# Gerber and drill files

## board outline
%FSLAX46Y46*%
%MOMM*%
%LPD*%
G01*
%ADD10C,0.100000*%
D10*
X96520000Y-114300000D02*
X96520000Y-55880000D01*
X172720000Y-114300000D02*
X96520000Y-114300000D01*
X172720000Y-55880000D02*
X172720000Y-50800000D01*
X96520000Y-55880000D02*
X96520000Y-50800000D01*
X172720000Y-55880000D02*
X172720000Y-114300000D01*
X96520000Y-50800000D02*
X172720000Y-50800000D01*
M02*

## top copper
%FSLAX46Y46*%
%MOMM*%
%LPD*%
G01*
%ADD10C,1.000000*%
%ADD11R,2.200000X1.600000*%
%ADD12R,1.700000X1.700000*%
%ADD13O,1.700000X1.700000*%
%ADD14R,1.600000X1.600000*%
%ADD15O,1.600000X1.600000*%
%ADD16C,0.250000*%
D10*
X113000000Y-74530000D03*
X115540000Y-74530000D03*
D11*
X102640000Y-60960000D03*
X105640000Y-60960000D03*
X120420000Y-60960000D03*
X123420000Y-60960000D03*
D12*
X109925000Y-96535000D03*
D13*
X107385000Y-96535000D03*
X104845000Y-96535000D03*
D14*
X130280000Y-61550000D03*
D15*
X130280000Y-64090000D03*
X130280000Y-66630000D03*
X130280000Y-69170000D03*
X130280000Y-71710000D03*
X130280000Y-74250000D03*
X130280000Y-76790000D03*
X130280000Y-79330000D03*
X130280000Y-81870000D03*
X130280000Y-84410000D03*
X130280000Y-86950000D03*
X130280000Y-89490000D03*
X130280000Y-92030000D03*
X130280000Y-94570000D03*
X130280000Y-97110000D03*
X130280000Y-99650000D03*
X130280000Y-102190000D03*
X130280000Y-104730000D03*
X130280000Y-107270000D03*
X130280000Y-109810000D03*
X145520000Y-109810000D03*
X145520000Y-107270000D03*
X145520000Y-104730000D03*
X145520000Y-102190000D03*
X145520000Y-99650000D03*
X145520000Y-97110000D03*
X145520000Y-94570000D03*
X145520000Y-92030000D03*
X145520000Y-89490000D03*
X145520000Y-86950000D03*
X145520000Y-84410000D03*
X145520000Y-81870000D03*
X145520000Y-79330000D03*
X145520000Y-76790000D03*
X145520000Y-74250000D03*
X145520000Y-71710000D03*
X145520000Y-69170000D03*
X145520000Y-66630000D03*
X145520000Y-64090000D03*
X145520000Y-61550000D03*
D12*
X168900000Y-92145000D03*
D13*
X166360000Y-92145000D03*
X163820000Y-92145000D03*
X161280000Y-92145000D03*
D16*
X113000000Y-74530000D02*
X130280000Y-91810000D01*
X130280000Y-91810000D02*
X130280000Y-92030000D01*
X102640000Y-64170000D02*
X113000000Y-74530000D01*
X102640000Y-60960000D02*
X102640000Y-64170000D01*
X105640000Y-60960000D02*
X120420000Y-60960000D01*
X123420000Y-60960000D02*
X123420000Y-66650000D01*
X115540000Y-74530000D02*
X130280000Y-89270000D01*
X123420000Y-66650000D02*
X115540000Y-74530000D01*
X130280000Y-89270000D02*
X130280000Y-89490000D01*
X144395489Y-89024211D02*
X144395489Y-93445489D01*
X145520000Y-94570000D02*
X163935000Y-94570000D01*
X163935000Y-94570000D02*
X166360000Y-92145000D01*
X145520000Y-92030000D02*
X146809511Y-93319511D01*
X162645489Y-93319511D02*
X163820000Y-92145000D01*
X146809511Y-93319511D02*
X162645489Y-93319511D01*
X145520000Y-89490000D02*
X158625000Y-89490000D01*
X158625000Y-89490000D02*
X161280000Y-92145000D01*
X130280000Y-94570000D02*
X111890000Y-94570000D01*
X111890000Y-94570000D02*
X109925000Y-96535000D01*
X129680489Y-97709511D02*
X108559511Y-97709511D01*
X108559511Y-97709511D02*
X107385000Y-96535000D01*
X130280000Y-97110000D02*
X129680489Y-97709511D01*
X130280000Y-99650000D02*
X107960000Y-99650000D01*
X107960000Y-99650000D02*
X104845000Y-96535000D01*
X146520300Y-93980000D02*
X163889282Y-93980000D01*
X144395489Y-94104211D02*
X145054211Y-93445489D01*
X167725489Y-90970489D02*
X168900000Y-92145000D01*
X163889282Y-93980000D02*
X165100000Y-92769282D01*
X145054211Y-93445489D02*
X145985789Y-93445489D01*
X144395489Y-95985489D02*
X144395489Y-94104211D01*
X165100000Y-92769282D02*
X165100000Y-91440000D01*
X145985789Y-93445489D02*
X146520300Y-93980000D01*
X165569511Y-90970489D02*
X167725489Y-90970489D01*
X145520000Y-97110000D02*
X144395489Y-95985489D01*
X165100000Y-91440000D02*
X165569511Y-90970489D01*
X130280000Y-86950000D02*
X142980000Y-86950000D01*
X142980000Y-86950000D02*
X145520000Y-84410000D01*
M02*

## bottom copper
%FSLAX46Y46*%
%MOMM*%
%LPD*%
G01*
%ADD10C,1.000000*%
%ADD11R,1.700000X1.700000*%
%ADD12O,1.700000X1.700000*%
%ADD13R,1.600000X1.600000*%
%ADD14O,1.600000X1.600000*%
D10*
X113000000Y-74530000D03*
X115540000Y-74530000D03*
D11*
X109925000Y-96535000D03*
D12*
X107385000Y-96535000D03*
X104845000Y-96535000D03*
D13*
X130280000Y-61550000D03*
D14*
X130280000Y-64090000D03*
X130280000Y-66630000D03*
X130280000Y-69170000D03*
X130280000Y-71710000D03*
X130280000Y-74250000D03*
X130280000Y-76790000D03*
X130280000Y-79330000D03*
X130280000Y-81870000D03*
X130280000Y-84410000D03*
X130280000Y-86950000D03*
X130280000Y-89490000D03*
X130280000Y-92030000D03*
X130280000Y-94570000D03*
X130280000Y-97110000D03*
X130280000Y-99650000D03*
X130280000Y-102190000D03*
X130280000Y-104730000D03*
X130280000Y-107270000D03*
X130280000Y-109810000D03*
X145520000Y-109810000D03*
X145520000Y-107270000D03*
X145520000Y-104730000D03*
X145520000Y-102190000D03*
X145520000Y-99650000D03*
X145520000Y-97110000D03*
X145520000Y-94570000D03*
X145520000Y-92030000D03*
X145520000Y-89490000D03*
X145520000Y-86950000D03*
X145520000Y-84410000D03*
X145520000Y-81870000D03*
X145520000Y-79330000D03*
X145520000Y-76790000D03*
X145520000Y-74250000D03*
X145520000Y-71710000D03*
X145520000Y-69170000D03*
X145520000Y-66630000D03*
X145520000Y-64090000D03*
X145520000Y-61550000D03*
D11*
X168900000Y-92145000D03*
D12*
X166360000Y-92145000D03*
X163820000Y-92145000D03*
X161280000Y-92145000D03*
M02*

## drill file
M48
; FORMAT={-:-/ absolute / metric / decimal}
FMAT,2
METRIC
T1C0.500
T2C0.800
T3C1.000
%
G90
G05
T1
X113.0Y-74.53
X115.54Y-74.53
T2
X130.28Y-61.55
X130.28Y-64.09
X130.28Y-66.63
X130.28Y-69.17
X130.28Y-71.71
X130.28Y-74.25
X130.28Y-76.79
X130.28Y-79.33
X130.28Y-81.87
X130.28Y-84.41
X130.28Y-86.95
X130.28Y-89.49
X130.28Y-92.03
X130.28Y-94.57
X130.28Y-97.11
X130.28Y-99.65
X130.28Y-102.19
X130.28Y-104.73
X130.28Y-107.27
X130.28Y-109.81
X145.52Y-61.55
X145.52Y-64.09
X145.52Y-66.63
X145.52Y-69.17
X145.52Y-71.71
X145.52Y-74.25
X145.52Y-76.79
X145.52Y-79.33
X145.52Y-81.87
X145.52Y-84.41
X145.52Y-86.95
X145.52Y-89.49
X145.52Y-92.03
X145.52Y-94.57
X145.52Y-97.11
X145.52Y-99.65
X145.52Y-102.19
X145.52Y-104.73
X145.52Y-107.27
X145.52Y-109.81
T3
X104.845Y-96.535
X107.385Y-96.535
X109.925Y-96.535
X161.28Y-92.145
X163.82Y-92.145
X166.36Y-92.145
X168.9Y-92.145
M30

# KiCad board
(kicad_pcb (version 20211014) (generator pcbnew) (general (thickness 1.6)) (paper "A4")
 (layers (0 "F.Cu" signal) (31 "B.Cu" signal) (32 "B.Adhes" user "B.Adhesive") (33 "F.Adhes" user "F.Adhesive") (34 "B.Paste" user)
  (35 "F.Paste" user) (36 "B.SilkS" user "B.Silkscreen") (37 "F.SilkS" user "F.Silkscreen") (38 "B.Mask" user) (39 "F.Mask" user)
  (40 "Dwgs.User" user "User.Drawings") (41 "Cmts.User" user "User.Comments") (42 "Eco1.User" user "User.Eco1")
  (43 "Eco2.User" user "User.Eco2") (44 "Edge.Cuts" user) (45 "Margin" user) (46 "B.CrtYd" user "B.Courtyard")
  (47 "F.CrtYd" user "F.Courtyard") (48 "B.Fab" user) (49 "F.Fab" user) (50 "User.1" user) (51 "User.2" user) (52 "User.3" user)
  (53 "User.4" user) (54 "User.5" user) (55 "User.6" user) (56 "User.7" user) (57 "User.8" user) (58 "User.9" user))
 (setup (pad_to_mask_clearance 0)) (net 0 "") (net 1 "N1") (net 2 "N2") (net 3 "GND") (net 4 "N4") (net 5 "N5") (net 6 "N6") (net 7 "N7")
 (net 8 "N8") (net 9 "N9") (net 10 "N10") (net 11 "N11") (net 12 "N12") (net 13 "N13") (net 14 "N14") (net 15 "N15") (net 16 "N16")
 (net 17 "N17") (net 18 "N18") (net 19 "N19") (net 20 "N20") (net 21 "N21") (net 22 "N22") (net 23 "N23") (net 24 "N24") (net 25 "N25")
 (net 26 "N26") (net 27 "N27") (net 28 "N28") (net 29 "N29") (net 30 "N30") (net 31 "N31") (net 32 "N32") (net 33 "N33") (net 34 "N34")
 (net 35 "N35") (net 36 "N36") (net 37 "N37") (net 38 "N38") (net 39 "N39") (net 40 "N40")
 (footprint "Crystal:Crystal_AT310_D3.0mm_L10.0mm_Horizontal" (layer "F.Cu") (at 113 74.53)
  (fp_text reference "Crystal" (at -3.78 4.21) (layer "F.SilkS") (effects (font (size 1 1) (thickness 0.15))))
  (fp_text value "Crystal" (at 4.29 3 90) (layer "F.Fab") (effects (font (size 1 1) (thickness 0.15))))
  (pad "1" thru_hole circle (at 0 0) (size 1 1) (drill 0.5) (layers *.Cu *.Mask) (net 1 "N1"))
  (pad "2" thru_hole circle (at 2.54 0) (size 1 1) (drill 0.5) (layers *.Cu *.Mask) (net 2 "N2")))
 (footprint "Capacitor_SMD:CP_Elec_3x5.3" (layer "F.Cu") (at 104.14 60.96)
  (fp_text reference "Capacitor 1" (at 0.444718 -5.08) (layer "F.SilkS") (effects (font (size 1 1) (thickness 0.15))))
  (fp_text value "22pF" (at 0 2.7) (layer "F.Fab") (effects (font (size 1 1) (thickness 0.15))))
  (pad "1" smd rect (at -1.5 0) (size 2.2 1.6) (layers "F.Cu" "F.Paste" "F.Mask") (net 1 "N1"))
  (pad "2" smd rect (at 1.5 0) (size 2.2 1.6) (layers "F.Cu" "F.Paste" "F.Mask") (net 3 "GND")))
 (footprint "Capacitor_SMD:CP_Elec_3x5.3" (layer "F.Cu") (at 121.92 60.96)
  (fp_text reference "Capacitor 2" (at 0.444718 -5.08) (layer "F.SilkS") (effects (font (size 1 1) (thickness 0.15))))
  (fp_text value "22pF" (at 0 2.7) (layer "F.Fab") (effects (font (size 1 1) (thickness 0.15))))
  (pad "1" smd rect (at -1.5 0) (size 2.2 1.6) (layers "F.Cu" "F.Paste" "F.Mask") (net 3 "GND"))
  (pad "2" smd rect (at 1.5 0) (size 2.2 1.6) (layers "F.Cu" "F.Paste" "F.Mask") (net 2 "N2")))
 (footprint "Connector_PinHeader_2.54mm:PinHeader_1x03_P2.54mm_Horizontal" (layer "F.Cu") (at 109.925 96.535 -90)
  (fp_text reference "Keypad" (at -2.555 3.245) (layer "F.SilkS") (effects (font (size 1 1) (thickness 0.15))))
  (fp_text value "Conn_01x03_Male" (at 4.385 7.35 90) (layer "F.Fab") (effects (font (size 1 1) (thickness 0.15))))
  (pad "1" thru_hole rect (at 0 0 270) (size 1.7 1.7) (drill 1) (layers *.Cu *.Mask) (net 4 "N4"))
  (pad "2" thru_hole oval (at 0 2.54 270) (size 1.7 1.7) (drill 1) (layers *.Cu *.Mask) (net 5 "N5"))
  (pad "3" thru_hole oval (at 0 5.08 270) (size 1.7 1.7) (drill 1) (layers *.Cu *.Mask) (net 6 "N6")))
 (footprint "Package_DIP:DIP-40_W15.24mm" (layer "F.Cu") (at 130.28 61.55)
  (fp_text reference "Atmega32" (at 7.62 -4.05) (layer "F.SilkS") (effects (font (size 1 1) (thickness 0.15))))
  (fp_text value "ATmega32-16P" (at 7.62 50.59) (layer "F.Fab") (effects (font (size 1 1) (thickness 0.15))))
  (pad "1" thru_hole rect (at 0 0) (size 1.6 1.6) (drill 0.8) (layers *.Cu *.Mask) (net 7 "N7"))
  (pad "2" thru_hole oval (at 0 2.54) (size 1.6 1.6) (drill 0.8) (layers *.Cu *.Mask) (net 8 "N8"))
  (pad "3" thru_hole oval (at 0 5.08) (size 1.6 1.6) (drill 0.8) (layers *.Cu *.Mask) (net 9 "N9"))
  (pad "4" thru_hole oval (at 0 7.62) (size 1.6 1.6) (drill 0.8) (layers *.Cu *.Mask) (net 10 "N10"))
  (pad "5" thru_hole oval (at 0 10.16) (size 1.6 1.6) (drill 0.8) (layers *.Cu *.Mask) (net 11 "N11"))
  (pad "6" thru_hole oval (at 0 12.7) (size 1.6 1.6) (drill 0.8) (layers *.Cu *.Mask) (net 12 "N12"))
  (pad "7" thru_hole oval (at 0 15.24) (size 1.6 1.6) (drill 0.8) (layers *.Cu *.Mask) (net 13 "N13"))
  (pad "8" thru_hole oval (at 0 17.78) (size 1.6 1.6) (drill 0.8) (layers *.Cu *.Mask) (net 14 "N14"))
  (pad "9" thru_hole oval (at 0 20.32) (size 1.6 1.6) (drill 0.8) (layers *.Cu *.Mask) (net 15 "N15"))
  (pad "10" thru_hole oval (at 0 22.86) (size 1.6 1.6) (drill 0.8) (layers *.Cu *.Mask) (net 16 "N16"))
  (pad "11" thru_hole oval (at 0 25.4) (size 1.6 1.6) (drill 0.8) (layers *.Cu *.Mask) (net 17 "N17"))
  (pad "12" thru_hole oval (at 0 27.94) (size 1.6 1.6) (drill 0.8) (layers *.Cu *.Mask) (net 2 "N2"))
  (pad "13" thru_hole oval (at 0 30.48) (size 1.6 1.6) (drill 0.8) (layers *.Cu *.Mask) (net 1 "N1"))
  (pad "14" thru_hole oval (at 0 33.02) (size 1.6 1.6) (drill 0.8) (layers *.Cu *.Mask) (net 4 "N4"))
  (pad "15" thru_hole oval (at 0 35.56) (size 1.6 1.6) (drill 0.8) (layers *.Cu *.Mask) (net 5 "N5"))
  (pad "16" thru_hole oval (at 0 38.1) (size 1.6 1.6) (drill 0.8) (layers *.Cu *.Mask) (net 6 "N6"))
  (pad "17" thru_hole oval (at 0 40.64) (size 1.6 1.6) (drill 0.8) (layers *.Cu *.Mask) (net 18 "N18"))
  (pad "18" thru_hole oval (at 0 43.18) (size 1.6 1.6) (drill 0.8) (layers *.Cu *.Mask) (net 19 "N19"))
  (pad "19" thru_hole oval (at 0 45.72) (size 1.6 1.6) (drill 0.8) (layers *.Cu *.Mask) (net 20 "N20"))
  (pad "20" thru_hole oval (at 0 48.26) (size 1.6 1.6) (drill 0.8) (layers *.Cu *.Mask) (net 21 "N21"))
  (pad "21" thru_hole oval (at 15.24 48.26) (size 1.6 1.6) (drill 0.8) (layers *.Cu *.Mask) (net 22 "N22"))
  (pad "22" thru_hole oval (at 15.24 45.72) (size 1.6 1.6) (drill 0.8) (layers *.Cu *.Mask) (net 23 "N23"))
  (pad "23" thru_hole oval (at 15.24 43.18) (size 1.6 1.6) (drill 0.8) (layers *.Cu *.Mask) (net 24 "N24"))
  (pad "24" thru_hole oval (at 15.24 40.64) (size 1.6 1.6) (drill 0.8) (layers *.Cu *.Mask) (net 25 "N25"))
  (pad "25" thru_hole oval (at 15.24 38.1) (size 1.6 1.6) (drill 0.8) (layers *.Cu *.Mask) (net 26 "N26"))
  (pad "26" thru_hole oval (at 15.24 35.56) (size 1.6 1.6) (drill 0.8) (layers *.Cu *.Mask) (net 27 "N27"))
  (pad "27" thru_hole oval (at 15.24 33.02) (size 1.6 1.6) (drill 0.8) (layers *.Cu *.Mask) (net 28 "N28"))
  (pad "28" thru_hole oval (at 15.24 30.48) (size 1.6 1.6) (drill 0.8) (layers *.Cu *.Mask) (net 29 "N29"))
  (pad "29" thru_hole oval (at 15.24 27.94) (size 1.6 1.6) (drill 0.8) (layers *.Cu *.Mask) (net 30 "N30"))
  (pad "30" thru_hole oval (at 15.24 25.4) (size 1.6 1.6) (drill 0.8) (layers *.Cu *.Mask) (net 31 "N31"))
  (pad "31" thru_hole oval (at 15.24 22.86) (size 1.6 1.6) (drill 0.8) (layers *.Cu *.Mask) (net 17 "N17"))
  (pad "32" thru_hole oval (at 15.24 20.32) (size 1.6 1.6) (drill 0.8) (layers *.Cu *.Mask) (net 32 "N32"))
  (pad "33" thru_hole oval (at 15.24 17.78) (size 1.6 1.6) (drill 0.8) (layers *.Cu *.Mask) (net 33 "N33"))
  (pad "34" thru_hole oval (at 15.24 15.24) (size 1.6 1.6) (drill 0.8) (layers *.Cu *.Mask) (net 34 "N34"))
  (pad "35" thru_hole oval (at 15.24 12.7) (size 1.6 1.6) (drill 0.8) (layers *.Cu *.Mask) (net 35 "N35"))
  (pad "36" thru_hole oval (at 15.24 10.16) (size 1.6 1.6) (drill 0.8) (layers *.Cu *.Mask) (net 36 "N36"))
  (pad "37" thru_hole oval (at 15.24 7.62) (size 1.6 1.6) (drill 0.8) (layers *.Cu *.Mask) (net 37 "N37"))
  (pad "38" thru_hole oval (at 15.24 5.08) (size 1.6 1.6) (drill 0.8) (layers *.Cu *.Mask) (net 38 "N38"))
  (pad "39" thru_hole oval (at 15.24 2.54) (size 1.6 1.6) (drill 0.8) (layers *.Cu *.Mask) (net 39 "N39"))
  (pad "40" thru_hole oval (at 15.24 0) (size 1.6 1.6) (drill 0.8) (layers *.Cu *.Mask) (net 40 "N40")))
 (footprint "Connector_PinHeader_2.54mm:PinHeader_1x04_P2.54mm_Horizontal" (layer "F.Cu") (at 168.9 92.145 -90)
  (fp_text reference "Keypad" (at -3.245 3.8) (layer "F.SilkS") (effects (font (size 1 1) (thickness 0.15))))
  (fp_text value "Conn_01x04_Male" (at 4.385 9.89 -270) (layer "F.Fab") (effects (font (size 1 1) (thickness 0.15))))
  (pad "1" thru_hole rect (at 0 0 270) (size 1.7 1.7) (drill 1) (layers *.Cu *.Mask) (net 27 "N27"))
  (pad "2" thru_hole oval (at 0 2.54 270) (size 1.7 1.7) (drill 1) (layers *.Cu *.Mask) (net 28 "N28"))
  (pad "3" thru_hole oval (at 0 5.08 270) (size 1.7 1.7) (drill 1) (layers *.Cu *.Mask) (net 29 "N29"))
  (pad "4" thru_hole oval (at 0 7.62 270) (size 1.7 1.7) (drill 1) (layers *.Cu *.Mask) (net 30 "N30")))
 (gr_line (start 96.52 114.3) (end 96.52 55.88) (layer "Edge.Cuts") (width 0.1))
 (gr_line (start 172.72 114.3) (end 96.52 114.3) (layer "Edge.Cuts") (width 0.1))
 (gr_line (start 172.72 55.88) (end 172.72 50.8) (layer "Edge.Cuts") (width 0.1))
 (gr_line (start 96.52 55.88) (end 96.52 50.8) (layer "Edge.Cuts") (width 0.1))
 (gr_line (start 172.72 55.88) (end 172.72 114.3) (layer "Edge.Cuts") (width 0.1))
 (gr_line (start 96.52 50.8) (end 172.72 50.8) (layer "Edge.Cuts") (width 0.1))
 (segment (start 113 74.53) (end 130.28 91.81) (width 0.25) (layer "F.Cu") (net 1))
 (segment (start 130.28 91.81) (end 130.28 92.03) (width 0.25) (layer "F.Cu") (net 1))
 (segment (start 102.64 64.17) (end 113 74.53) (width 0.25) (layer "F.Cu") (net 1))
 (segment (start 102.64 60.96) (end 102.64 64.17) (width 0.25) (layer "F.Cu") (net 1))
 (segment (start 105.64 60.96) (end 120.42 60.96) (width 0.25) (layer "F.Cu") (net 3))
 (segment (start 123.42 60.96) (end 123.42 66.65) (width 0.25) (layer "F.Cu") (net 2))
 (segment (start 115.54 74.53) (end 130.28 89.27) (width 0.25) (layer "F.Cu") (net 2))
 (segment (start 123.42 66.65) (end 115.54 74.53) (width 0.25) (layer "F.Cu") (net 2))
 (segment (start 130.28 89.27) (end 130.28 89.49) (width 0.25) (layer "F.Cu") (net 2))
 (segment (start 144.395489 89.024211) (end 144.395489 93.445489) (width 0.25) (layer "F.Cu") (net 28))
 (segment (start 145.52 94.57) (end 163.935 94.57) (width 0.25) (layer "F.Cu") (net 28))
 (segment (start 163.935 94.57) (end 166.36 92.145) (width 0.25) (layer "F.Cu") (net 28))
 (segment (start 145.52 92.03) (end 146.809511 93.319511) (width 0.25) (layer "F.Cu") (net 29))
 (segment (start 162.645489 93.319511) (end 163.82 92.145) (width 0.25) (layer "F.Cu") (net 29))
 (segment (start 146.809511 93.319511) (end 162.645489 93.319511) (width 0.25) (layer "F.Cu") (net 29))
 (segment (start 145.52 89.49) (end 158.625 89.49) (width 0.25) (layer "F.Cu") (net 30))
 (segment (start 158.625 89.49) (end 161.28 92.145) (width 0.25) (layer "F.Cu") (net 30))
 (segment (start 130.28 94.57) (end 111.89 94.57) (width 0.25) (layer "F.Cu") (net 4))
 (segment (start 111.89 94.57) (end 109.925 96.535) (width 0.25) (layer "F.Cu") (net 4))
 (segment (start 129.680489 97.709511) (end 108.559511 97.709511) (width 0.25) (layer "F.Cu") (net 5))
 (segment (start 108.559511 97.709511) (end 107.385 96.535) (width 0.25) (layer "F.Cu") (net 5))
 (segment (start 130.28 97.11) (end 129.680489 97.709511) (width 0.25) (layer "F.Cu") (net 5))
 (segment (start 130.28 99.65) (end 107.96 99.65) (width 0.25) (layer "F.Cu") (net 6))
 (segment (start 107.96 99.65) (end 104.845 96.535) (width 0.25) (layer "F.Cu") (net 6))
 (segment (start 146.5203 93.98) (end 163.889282 93.98) (width 0.25) (layer "F.Cu") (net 27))
 (segment (start 144.395489 94.104211) (end 145.054211 93.445489) (width 0.25) (layer "F.Cu") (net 27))
 (segment (start 167.725489 90.970489) (end 168.9 92.145) (width 0.25) (layer "F.Cu") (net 27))
 (segment (start 163.889282 93.98) (end 165.1 92.769282) (width 0.25) (layer "F.Cu") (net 27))
 (segment (start 145.054211 93.445489) (end 145.985789 93.445489) (width 0.25) (layer "F.Cu") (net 27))
 (segment (start 144.395489 95.985489) (end 144.395489 94.104211) (width 0.25) (layer "F.Cu") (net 27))
 (segment (start 165.1 92.769282) (end 165.1 91.44) (width 0.25) (layer "F.Cu") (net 27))
 (segment (start 145.985789 93.445489) (end 146.5203 93.98) (width 0.25) (layer "F.Cu") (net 27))
 (segment (start 165.569511 90.970489) (end 167.725489 90.970489) (width 0.25) (layer "F.Cu") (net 27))
 (segment (start 145.52 97.11) (end 144.395489 95.985489) (width 0.25) (layer "F.Cu") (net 27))
 (segment (start 165.1 91.44) (end 165.569511 90.970489) (width 0.25) (layer "F.Cu") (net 27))
 (segment (start 130.28 86.95) (end 142.98 86.95) (width 0.25) (layer "F.Cu") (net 17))
 (segment (start 142.98 86.95) (end 145.52 84.41) (width 0.25) (layer "F.Cu") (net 17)))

